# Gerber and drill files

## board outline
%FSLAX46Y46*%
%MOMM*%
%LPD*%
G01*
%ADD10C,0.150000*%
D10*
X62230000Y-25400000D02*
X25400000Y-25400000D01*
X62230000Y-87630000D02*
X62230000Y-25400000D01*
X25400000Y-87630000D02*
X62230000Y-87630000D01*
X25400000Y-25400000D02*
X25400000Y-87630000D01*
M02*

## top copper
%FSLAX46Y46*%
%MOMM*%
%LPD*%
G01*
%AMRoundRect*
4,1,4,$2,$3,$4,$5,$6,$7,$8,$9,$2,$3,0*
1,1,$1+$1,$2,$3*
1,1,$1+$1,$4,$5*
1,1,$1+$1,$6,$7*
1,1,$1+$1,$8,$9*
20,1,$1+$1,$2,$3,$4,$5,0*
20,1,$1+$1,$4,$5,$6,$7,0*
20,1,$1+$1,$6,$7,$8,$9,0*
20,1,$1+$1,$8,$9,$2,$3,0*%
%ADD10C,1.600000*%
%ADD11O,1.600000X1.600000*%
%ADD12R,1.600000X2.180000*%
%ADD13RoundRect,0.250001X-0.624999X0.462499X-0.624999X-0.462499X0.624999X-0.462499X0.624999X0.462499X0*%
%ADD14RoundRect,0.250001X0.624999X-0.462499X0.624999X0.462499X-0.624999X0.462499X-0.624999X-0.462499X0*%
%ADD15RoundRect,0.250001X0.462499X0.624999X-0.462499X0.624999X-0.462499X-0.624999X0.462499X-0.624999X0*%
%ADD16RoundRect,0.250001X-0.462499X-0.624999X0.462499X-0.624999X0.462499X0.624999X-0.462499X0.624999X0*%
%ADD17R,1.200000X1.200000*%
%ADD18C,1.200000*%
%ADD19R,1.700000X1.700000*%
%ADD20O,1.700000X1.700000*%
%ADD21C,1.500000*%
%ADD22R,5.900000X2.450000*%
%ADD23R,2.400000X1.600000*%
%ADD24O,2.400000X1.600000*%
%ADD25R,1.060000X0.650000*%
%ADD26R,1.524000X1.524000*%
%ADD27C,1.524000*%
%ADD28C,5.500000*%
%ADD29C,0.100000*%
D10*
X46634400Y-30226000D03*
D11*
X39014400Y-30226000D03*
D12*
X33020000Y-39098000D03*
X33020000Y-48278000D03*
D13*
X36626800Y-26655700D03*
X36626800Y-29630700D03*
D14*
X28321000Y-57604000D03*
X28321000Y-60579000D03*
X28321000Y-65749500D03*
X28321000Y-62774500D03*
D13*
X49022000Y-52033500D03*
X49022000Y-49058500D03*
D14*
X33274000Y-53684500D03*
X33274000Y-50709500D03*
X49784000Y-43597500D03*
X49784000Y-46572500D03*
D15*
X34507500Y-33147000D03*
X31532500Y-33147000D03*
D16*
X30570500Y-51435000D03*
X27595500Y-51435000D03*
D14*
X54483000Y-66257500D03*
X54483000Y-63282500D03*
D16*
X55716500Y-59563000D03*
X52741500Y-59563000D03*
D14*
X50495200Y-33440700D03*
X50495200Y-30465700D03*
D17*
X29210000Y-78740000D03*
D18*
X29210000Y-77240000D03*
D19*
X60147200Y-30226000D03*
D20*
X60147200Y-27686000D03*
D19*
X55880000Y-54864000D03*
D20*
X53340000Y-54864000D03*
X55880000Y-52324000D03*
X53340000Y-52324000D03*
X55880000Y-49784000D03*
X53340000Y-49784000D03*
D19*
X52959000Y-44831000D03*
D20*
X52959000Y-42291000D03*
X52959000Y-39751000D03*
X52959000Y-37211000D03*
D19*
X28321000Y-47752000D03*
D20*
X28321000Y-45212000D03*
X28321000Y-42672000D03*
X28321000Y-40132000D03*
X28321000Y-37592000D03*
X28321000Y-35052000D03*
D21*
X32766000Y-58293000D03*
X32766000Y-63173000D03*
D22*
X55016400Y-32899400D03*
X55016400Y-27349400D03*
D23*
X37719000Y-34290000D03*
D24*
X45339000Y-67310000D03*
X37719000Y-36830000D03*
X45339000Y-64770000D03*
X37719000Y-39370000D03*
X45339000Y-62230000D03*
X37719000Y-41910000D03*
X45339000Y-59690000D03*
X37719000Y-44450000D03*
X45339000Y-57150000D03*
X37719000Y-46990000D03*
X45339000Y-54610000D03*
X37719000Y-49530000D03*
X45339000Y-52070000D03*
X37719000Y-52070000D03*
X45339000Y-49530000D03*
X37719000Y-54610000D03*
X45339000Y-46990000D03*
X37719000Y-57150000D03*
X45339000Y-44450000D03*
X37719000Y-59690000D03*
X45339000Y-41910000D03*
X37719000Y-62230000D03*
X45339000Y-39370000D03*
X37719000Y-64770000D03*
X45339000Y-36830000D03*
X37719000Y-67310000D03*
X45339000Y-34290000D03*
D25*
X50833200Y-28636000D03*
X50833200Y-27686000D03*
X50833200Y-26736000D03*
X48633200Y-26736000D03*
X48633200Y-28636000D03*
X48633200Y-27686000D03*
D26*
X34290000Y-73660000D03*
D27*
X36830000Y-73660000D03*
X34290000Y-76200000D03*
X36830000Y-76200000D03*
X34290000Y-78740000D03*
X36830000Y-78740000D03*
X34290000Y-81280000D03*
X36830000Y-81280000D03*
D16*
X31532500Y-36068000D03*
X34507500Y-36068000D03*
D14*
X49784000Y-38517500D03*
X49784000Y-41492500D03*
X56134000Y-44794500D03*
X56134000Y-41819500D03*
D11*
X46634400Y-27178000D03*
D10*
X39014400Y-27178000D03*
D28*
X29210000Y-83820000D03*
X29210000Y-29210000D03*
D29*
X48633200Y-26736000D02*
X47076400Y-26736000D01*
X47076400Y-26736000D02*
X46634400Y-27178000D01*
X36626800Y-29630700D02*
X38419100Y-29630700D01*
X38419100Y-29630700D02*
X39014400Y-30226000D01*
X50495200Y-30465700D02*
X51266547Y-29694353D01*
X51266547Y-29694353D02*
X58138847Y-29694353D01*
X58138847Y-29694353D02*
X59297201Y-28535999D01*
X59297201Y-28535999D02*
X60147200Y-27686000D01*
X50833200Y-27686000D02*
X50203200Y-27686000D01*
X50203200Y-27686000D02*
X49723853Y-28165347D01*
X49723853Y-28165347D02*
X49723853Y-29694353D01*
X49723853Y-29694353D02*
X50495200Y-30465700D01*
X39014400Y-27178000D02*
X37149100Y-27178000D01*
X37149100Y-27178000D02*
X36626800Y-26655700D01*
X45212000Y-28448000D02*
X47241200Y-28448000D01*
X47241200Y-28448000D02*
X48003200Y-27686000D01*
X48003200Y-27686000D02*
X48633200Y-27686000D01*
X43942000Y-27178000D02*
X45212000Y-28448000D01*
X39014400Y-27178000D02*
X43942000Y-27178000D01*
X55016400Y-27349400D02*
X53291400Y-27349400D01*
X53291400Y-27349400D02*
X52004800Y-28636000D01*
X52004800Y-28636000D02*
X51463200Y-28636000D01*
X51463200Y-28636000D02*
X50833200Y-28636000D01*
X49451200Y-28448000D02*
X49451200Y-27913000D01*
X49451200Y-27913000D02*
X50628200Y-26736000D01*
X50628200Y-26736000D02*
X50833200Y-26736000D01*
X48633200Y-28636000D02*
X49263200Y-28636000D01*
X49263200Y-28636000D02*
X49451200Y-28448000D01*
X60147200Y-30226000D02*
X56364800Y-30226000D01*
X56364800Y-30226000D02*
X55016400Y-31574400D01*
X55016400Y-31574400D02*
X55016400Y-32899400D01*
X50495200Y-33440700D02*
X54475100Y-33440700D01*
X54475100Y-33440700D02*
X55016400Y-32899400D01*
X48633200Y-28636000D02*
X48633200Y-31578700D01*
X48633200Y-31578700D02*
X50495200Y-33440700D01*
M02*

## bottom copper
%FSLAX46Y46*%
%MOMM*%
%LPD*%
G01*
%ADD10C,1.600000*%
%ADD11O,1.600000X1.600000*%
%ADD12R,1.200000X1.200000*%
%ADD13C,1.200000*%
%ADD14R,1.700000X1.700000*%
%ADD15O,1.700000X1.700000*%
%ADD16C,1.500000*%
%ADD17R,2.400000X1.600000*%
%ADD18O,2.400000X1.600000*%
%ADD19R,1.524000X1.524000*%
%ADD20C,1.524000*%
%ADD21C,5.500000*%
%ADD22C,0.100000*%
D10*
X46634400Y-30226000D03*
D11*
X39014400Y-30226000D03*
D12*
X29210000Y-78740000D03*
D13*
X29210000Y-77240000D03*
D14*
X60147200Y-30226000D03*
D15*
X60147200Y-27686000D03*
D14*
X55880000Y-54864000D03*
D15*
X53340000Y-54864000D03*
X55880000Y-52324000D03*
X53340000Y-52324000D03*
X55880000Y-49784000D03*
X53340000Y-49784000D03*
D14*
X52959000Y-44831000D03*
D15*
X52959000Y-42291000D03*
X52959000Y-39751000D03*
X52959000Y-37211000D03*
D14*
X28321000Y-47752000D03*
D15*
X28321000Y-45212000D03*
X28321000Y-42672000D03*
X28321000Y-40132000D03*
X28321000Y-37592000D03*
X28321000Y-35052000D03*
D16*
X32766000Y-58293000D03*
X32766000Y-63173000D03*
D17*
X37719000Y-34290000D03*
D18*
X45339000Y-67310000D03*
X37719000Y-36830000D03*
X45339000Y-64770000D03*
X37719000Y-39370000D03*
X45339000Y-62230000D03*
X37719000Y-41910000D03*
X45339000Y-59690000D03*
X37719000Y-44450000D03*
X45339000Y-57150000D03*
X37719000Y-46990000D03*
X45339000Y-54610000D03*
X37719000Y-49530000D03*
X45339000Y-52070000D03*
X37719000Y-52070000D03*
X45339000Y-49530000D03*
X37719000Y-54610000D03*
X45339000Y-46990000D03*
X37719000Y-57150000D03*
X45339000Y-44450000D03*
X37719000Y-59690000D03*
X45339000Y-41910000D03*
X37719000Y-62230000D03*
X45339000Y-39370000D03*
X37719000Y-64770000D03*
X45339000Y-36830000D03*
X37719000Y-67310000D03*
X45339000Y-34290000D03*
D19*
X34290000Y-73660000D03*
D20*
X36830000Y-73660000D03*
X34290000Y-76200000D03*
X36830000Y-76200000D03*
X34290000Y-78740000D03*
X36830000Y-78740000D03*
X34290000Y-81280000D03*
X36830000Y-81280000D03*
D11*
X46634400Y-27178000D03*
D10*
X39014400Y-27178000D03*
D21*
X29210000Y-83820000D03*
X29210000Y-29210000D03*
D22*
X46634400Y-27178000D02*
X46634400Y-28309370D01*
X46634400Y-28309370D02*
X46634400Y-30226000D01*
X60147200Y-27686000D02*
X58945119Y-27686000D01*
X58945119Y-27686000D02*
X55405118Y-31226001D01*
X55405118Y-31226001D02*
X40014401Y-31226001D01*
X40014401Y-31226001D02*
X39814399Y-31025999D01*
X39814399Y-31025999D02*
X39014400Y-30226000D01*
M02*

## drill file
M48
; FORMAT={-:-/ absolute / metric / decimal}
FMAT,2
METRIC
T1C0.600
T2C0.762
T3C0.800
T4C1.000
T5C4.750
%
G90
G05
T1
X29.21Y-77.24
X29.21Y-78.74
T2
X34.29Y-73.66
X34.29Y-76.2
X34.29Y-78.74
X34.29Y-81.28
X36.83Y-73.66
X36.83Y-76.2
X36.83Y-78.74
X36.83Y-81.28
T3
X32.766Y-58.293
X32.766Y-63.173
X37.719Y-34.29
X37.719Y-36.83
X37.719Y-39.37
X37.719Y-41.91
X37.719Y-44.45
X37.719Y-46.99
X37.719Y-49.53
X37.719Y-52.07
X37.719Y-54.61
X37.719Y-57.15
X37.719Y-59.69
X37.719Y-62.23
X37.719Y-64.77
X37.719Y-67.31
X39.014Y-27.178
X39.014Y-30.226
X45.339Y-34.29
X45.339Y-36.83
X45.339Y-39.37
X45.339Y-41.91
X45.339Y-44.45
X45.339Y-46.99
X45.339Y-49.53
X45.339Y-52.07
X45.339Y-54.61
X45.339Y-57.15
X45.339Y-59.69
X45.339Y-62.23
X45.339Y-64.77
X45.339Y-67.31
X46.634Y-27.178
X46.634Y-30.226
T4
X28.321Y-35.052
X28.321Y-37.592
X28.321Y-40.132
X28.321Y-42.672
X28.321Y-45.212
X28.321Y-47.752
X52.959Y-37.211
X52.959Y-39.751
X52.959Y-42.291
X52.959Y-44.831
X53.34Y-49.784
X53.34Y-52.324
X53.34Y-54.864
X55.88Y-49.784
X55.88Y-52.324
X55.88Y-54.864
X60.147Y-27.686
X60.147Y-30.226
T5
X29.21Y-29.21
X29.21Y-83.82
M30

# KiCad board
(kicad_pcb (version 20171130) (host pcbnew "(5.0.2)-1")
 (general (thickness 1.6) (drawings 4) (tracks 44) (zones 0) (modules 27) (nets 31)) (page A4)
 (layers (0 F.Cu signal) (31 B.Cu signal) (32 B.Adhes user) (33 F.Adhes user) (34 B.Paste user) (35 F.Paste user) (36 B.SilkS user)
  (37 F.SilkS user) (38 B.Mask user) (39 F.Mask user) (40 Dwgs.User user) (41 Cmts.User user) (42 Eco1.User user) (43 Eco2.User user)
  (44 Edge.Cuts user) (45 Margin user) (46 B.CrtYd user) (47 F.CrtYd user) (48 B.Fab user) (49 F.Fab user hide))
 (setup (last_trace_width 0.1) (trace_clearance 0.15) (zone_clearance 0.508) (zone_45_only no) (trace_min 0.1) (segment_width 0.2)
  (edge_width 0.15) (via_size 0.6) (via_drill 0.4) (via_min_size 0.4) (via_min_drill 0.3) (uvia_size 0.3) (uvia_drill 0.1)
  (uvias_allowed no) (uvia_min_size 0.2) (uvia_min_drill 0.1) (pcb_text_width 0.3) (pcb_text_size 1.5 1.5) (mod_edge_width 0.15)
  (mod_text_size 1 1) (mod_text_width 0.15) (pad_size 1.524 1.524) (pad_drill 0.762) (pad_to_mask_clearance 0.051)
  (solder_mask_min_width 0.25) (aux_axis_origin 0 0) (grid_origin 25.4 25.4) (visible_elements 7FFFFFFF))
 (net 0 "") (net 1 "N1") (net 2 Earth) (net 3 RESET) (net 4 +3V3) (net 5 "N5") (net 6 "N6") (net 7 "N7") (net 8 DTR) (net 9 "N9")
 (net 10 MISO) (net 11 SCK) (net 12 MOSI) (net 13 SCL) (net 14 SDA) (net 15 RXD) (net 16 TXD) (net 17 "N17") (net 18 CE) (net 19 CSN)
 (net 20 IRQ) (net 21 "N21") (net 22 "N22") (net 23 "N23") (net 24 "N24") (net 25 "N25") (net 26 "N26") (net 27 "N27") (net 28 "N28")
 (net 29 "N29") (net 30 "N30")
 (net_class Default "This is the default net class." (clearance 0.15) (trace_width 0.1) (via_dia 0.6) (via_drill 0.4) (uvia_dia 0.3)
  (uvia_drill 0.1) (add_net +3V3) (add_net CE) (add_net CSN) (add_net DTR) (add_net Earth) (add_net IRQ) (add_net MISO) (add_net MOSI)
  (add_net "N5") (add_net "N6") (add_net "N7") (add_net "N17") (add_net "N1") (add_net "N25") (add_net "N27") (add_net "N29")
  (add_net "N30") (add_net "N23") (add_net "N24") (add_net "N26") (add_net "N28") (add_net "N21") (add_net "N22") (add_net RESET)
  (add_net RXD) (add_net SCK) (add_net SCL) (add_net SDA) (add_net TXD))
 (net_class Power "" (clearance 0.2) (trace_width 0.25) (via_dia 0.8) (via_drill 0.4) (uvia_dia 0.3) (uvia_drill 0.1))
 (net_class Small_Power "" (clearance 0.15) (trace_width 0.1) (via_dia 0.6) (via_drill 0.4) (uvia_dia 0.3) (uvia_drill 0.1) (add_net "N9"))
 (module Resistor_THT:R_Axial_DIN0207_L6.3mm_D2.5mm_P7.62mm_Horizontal (layer F.Cu) (at 46.6344 30.226 180)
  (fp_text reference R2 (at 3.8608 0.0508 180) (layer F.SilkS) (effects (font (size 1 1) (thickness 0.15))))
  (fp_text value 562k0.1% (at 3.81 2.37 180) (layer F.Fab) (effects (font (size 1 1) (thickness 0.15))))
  (pad 1 thru_hole circle (at 0 0 180) (size 1.6 1.6) (drill 0.8) (layers *.Cu *.Mask) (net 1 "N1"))
  (pad 2 thru_hole oval (at 7.62 0 180) (size 1.6 1.6) (drill 0.8) (layers *.Cu *.Mask) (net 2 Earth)))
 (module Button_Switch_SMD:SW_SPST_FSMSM (layer F.Cu) (at 33.02 43.688 270)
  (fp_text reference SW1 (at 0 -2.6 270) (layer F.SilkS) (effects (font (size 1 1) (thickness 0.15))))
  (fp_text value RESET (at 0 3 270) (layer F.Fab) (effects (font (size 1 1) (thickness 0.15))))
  (pad 1 smd rect (at -4.59 0 270) (size 2.18 1.6) (layers F.Cu F.Paste F.Mask) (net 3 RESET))
  (pad 2 smd rect (at 4.59 0 270) (size 2.18 1.6) (layers F.Cu F.Paste F.Mask) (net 2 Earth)))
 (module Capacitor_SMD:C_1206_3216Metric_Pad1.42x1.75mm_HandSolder (layer F.Cu) (at 36.6268 28.1432 270)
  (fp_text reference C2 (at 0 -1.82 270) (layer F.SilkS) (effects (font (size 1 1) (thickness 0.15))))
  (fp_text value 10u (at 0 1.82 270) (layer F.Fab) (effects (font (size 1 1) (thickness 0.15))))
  (pad 1 smd roundrect (at -1.4875 0 270) (size 1.425 1.75) (layers F.Cu F.Paste F.Mask) (roundrect_rratio 0.175439) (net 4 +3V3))
  (pad 2 smd roundrect (at 1.4875 0 270) (size 1.425 1.75) (layers F.Cu F.Paste F.Mask) (roundrect_rratio 0.175439) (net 2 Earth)))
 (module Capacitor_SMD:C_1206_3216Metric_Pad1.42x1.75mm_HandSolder (layer F.Cu) (at 28.321 59.0915 90)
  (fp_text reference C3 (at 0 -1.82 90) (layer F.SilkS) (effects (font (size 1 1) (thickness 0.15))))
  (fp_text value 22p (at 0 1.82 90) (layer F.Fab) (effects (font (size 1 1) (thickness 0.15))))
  (pad 2 smd roundrect (at 1.4875 0 90) (size 1.425 1.75) (layers F.Cu F.Paste F.Mask) (roundrect_rratio 0.175439) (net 2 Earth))
  (pad 1 smd roundrect (at -1.4875 0 90) (size 1.425 1.75) (layers F.Cu F.Paste F.Mask) (roundrect_rratio 0.175439) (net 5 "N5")))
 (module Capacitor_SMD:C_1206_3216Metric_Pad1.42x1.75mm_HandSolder (layer F.Cu) (at 28.321 64.262 90)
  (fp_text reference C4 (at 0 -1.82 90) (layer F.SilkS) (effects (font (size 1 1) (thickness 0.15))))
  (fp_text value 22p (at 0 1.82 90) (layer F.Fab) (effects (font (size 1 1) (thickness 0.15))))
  (pad 1 smd roundrect (at -1.4875 0 90) (size 1.425 1.75) (layers F.Cu F.Paste F.Mask) (roundrect_rratio 0.175439) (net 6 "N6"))
  (pad 2 smd roundrect (at 1.4875 0 90) (size 1.425 1.75) (layers F.Cu F.Paste F.Mask) (roundrect_rratio 0.175439) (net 2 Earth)))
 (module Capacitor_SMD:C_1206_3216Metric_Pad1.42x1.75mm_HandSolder (layer F.Cu) (at 49.022 50.546 270)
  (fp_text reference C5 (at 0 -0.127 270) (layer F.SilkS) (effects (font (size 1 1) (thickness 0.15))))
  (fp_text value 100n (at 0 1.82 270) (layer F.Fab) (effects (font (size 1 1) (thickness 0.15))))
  (pad 2 smd roundrect (at 1.4875 0 270) (size 1.425 1.75) (layers F.Cu F.Paste F.Mask) (roundrect_rratio 0.175439) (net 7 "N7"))
  (pad 1 smd roundrect (at -1.4875 0 270) (size 1.425 1.75) (layers F.Cu F.Paste F.Mask) (roundrect_rratio 0.175439) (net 2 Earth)))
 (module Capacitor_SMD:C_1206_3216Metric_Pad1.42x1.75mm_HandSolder (layer F.Cu) (at 33.274 52.197 90)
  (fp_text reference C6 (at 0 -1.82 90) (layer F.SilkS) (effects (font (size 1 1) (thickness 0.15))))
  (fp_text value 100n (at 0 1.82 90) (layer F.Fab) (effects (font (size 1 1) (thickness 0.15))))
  (pad 1 smd roundrect (at -1.4875 0 90) (size 1.425 1.75) (layers F.Cu F.Paste F.Mask) (roundrect_rratio 0.175439) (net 4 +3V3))
  (pad 2 smd roundrect (at 1.4875 0 90) (size 1.425 1.75) (layers F.Cu F.Paste F.Mask) (roundrect_rratio 0.175439) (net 2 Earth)))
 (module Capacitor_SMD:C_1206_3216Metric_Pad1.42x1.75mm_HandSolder (layer F.Cu) (at 49.784 45.085 90)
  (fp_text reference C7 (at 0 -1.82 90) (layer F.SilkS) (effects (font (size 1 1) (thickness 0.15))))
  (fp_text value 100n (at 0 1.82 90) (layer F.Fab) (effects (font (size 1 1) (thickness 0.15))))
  (pad 2 smd roundrect (at 1.4875 0 90) (size 1.425 1.75) (layers F.Cu F.Paste F.Mask) (roundrect_rratio 0.175439) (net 4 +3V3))
  (pad 1 smd roundrect (at -1.4875 0 90) (size 1.425 1.75) (layers F.Cu F.Paste F.Mask) (roundrect_rratio 0.175439) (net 2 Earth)))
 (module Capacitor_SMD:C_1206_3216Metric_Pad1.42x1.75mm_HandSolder (layer F.Cu) (at 33.02 33.147 180)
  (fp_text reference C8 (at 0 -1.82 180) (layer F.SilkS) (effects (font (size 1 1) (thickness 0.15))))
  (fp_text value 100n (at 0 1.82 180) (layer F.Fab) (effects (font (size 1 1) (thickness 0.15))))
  (pad 1 smd roundrect (at -1.4875 0 180) (size 1.425 1.75) (layers F.Cu F.Paste F.Mask) (roundrect_rratio 0.175439) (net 3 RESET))
  (pad 2 smd roundrect (at 1.4875 0 180) (size 1.425 1.75) (layers F.Cu F.Paste F.Mask) (roundrect_rratio 0.175439) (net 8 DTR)))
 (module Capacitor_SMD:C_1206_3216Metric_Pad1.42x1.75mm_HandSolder (layer F.Cu) (at 29.083 51.435)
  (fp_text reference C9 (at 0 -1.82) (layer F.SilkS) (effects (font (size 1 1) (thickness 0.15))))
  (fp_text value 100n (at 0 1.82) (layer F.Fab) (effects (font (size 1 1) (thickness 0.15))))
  (pad 2 smd roundrect (at 1.4875 0) (size 1.425 1.75) (layers F.Cu F.Paste F.Mask) (roundrect_rratio 0.175439) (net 2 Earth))
  (pad 1 smd roundrect (at -1.4875 0) (size 1.425 1.75) (layers F.Cu F.Paste F.Mask) (roundrect_rratio 0.175439) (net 4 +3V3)))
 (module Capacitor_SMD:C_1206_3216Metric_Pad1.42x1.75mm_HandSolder (layer F.Cu) (at 54.483 64.77 90)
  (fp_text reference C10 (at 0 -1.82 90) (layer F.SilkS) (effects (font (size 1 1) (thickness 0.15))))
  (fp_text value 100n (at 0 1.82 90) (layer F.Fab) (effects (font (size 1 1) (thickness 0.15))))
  (pad 1 smd roundrect (at -1.4875 0 90) (size 1.425 1.75) (layers F.Cu F.Paste F.Mask) (roundrect_rratio 0.175439) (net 4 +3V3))
  (pad 2 smd roundrect (at 1.4875 0 90) (size 1.425 1.75) (layers F.Cu F.Paste F.Mask) (roundrect_rratio 0.175439) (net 2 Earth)))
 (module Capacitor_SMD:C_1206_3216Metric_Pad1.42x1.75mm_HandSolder (layer F.Cu) (at 54.229 59.563)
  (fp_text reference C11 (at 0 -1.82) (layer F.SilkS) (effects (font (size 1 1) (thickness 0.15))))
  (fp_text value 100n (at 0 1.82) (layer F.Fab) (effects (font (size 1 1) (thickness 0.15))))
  (pad 2 smd roundrect (at 1.4875 0) (size 1.425 1.75) (layers F.Cu F.Paste F.Mask) (roundrect_rratio 0.175439) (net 2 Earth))
  (pad 1 smd roundrect (at -1.4875 0) (size 1.425 1.75) (layers F.Cu F.Paste F.Mask) (roundrect_rratio 0.175439) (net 4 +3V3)))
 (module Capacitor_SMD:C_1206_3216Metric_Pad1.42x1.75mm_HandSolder (layer F.Cu) (at 50.4952 31.9532 90)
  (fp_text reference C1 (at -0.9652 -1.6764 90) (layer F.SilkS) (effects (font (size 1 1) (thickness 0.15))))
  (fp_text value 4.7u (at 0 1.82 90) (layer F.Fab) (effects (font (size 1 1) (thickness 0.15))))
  (pad 1 smd roundrect (at -1.4875 0 90) (size 1.425 1.75) (layers F.Cu F.Paste F.Mask) (roundrect_rratio 0.175439) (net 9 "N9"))
  (pad 2 smd roundrect (at 1.4875 0 90) (size 1.425 1.75) (layers F.Cu F.Paste F.Mask) (roundrect_rratio 0.175439) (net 2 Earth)))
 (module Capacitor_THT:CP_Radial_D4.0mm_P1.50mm (layer F.Cu) (at 29.21 78.74 90)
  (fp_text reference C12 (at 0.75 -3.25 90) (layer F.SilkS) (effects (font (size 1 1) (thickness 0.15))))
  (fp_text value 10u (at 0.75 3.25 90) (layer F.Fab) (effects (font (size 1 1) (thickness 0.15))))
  (pad 1 thru_hole rect (at 0 0 90) (size 1.2 1.2) (drill 0.6) (layers *.Cu *.Mask) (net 4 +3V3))
  (pad 2 thru_hole circle (at 1.5 0 90) (size 1.2 1.2) (drill 0.6) (layers *.Cu *.Mask) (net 2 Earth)))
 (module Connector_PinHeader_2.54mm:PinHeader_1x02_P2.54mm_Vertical (layer F.Cu) (at 60.1472 30.226 180)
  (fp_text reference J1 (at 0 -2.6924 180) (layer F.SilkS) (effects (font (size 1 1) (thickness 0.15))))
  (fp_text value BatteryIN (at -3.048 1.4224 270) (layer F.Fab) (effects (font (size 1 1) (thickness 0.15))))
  (pad 1 thru_hole rect (at 0 0 180) (size 1.7 1.7) (drill 1) (layers *.Cu *.Mask) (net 9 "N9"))
  (pad 2 thru_hole oval (at 0 2.54 180) (size 1.7 1.7) (drill 1) (layers *.Cu *.Mask) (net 2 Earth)))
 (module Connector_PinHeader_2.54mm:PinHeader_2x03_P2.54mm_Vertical (layer F.Cu) (at 55.88 54.864 180)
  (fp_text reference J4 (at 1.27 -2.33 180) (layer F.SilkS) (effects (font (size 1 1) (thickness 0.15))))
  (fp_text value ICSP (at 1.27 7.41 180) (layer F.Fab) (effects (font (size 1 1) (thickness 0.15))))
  (pad 1 thru_hole rect (at 0 0 180) (size 1.7 1.7) (drill 1) (layers *.Cu *.Mask) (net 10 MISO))
  (pad 2 thru_hole oval (at 2.54 0 180) (size 1.7 1.7) (drill 1) (layers *.Cu *.Mask) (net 4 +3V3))
  (pad 3 thru_hole oval (at 0 2.54 180) (size 1.7 1.7) (drill 1) (layers *.Cu *.Mask) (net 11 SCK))
  (pad 4 thru_hole oval (at 2.54 2.54 180) (size 1.7 1.7) (drill 1) (layers *.Cu *.Mask) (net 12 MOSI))
  (pad 5 thru_hole oval (at 0 5.08 180) (size 1.7 1.7) (drill 1) (layers *.Cu *.Mask) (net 3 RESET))
  (pad 6 thru_hole oval (at 2.54 5.08 180) (size 1.7 1.7) (drill 1) (layers *.Cu *.Mask) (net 2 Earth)))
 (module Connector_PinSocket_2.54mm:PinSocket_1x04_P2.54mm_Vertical (layer F.Cu) (at 52.959 44.831 180)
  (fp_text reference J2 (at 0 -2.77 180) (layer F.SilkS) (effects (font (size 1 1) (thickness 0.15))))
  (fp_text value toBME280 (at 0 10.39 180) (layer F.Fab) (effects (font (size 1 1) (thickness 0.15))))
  (pad 1 thru_hole rect (at 0 0 180) (size 1.7 1.7) (drill 1) (layers *.Cu *.Mask) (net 4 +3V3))
  (pad 2 thru_hole oval (at 0 2.54 180) (size 1.7 1.7) (drill 1) (layers *.Cu *.Mask) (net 2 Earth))
  (pad 3 thru_hole oval (at 0 5.08 180) (size 1.7 1.7) (drill 1) (layers *.Cu *.Mask) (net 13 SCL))
  (pad 4 thru_hole oval (at 0 7.62 180) (size 1.7 1.7) (drill 1) (layers *.Cu *.Mask) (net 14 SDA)))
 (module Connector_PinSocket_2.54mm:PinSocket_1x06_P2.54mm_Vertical (layer F.Cu) (at 28.321 47.752 180)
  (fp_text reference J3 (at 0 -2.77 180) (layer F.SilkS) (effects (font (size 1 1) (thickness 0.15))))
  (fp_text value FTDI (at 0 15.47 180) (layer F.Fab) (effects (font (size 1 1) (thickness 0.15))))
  (pad 1 thru_hole rect (at 0 0 180) (size 1.7 1.7) (drill 1) (layers *.Cu *.Mask) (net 2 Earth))
  (pad 2 thru_hole oval (at 0 2.54 180) (size 1.7 1.7) (drill 1) (layers *.Cu *.Mask) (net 2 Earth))
  (pad 3 thru_hole oval (at 0 5.08 180) (size 1.7 1.7) (drill 1) (layers *.Cu *.Mask) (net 4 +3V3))
  (pad 4 thru_hole oval (at 0 7.62 180) (size 1.7 1.7) (drill 1) (layers *.Cu *.Mask) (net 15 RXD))
  (pad 5 thru_hole oval (at 0 10.16 180) (size 1.7 1.7) (drill 1) (layers *.Cu *.Mask) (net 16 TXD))
  (pad 6 thru_hole oval (at 0 12.7 180) (size 1.7 1.7) (drill 1) (layers *.Cu *.Mask) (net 8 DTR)))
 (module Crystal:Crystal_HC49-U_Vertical (layer F.Cu) (at 32.766 58.293 270)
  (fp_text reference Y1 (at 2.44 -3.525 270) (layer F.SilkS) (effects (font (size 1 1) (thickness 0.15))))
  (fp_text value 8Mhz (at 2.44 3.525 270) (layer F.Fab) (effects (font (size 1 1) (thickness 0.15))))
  (pad 1 thru_hole circle (at 0 0 270) (size 1.5 1.5) (drill 0.8) (layers *.Cu *.Mask) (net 5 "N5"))
  (pad 2 thru_hole circle (at 4.88 0 270) (size 1.5 1.5) (drill 0.8) (layers *.Cu *.Mask) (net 6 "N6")))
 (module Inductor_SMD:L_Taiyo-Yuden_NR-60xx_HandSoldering (layer F.Cu) (at 55.0164 30.1244 90)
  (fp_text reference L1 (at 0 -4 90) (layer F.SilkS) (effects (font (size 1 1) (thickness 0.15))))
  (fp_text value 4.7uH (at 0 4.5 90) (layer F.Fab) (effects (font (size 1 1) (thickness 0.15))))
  (pad 1 smd rect (at -2.775 0 90) (size 2.45 5.9) (layers F.Cu F.Paste F.Mask) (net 9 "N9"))
  (pad 2 smd rect (at 2.775 0 90) (size 2.45 5.9) (layers F.Cu F.Paste F.Mask) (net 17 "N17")))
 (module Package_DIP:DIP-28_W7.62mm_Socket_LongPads (layer F.Cu) (at 37.719 34.29)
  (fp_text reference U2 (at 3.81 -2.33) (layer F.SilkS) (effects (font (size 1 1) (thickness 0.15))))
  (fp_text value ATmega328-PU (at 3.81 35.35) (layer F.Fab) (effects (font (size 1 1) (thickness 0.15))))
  (pad 1 thru_hole rect (at 0 0) (size 2.4 1.6) (drill 0.8) (layers *.Cu *.Mask) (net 3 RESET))
  (pad 15 thru_hole oval (at 7.62 33.02) (size 2.4 1.6) (drill 0.8) (layers *.Cu *.Mask) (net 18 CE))
  (pad 2 thru_hole oval (at 0 2.54) (size 2.4 1.6) (drill 0.8) (layers *.Cu *.Mask) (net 15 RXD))
  (pad 16 thru_hole oval (at 7.62 30.48) (size 2.4 1.6) (drill 0.8) (layers *.Cu *.Mask) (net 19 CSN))
  (pad 3 thru_hole oval (at 0 5.08) (size 2.4 1.6) (drill 0.8) (layers *.Cu *.Mask) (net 16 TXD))
  (pad 17 thru_hole oval (at 7.62 27.94) (size 2.4 1.6) (drill 0.8) (layers *.Cu *.Mask) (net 12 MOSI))
  (pad 4 thru_hole oval (at 0 7.62) (size 2.4 1.6) (drill 0.8) (layers *.Cu *.Mask) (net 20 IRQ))
  (pad 18 thru_hole oval (at 7.62 25.4) (size 2.4 1.6) (drill 0.8) (layers *.Cu *.Mask) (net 10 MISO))
  (pad 5 thru_hole oval (at 0 10.16) (size 2.4 1.6) (drill 0.8) (layers *.Cu *.Mask) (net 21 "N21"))
  (pad 19 thru_hole oval (at 7.62 22.86) (size 2.4 1.6) (drill 0.8) (layers *.Cu *.Mask) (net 11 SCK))
  (pad 6 thru_hole oval (at 0 12.7) (size 2.4 1.6) (drill 0.8) (layers *.Cu *.Mask) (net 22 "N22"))
  (pad 20 thru_hole oval (at 7.62 20.32) (size 2.4 1.6) (drill 0.8) (layers *.Cu *.Mask) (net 4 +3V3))
  (pad 7 thru_hole oval (at 0 15.24) (size 2.4 1.6) (drill 0.8) (layers *.Cu *.Mask) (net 4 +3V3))
  (pad 21 thru_hole oval (at 7.62 17.78) (size 2.4 1.6) (drill 0.8) (layers *.Cu *.Mask) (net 7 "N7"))
  (pad 8 thru_hole oval (at 0 17.78) (size 2.4 1.6) (drill 0.8) (layers *.Cu *.Mask) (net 2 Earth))
  (pad 22 thru_hole oval (at 7.62 15.24) (size 2.4 1.6) (drill 0.8) (layers *.Cu *.Mask) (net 2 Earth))
  (pad 9 thru_hole oval (at 0 20.32) (size 2.4 1.6) (drill 0.8) (layers *.Cu *.Mask) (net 5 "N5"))
  (pad 23 thru_hole oval (at 7.62 12.7) (size 2.4 1.6) (drill 0.8) (layers *.Cu *.Mask) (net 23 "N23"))
  (pad 10 thru_hole oval (at 0 22.86) (size 2.4 1.6) (drill 0.8) (layers *.Cu *.Mask) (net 6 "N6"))
  (pad 24 thru_hole oval (at 7.62 10.16) (size 2.4 1.6) (drill 0.8) (layers *.Cu *.Mask) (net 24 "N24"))
  (pad 11 thru_hole oval (at 0 25.4) (size 2.4 1.6) (drill 0.8) (layers *.Cu *.Mask) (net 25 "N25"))
  (pad 25 thru_hole oval (at 7.62 7.62) (size 2.4 1.6) (drill 0.8) (layers *.Cu *.Mask) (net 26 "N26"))
  (pad 12 thru_hole oval (at 0 27.94) (size 2.4 1.6) (drill 0.8) (layers *.Cu *.Mask) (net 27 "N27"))
  (pad 26 thru_hole oval (at 7.62 5.08) (size 2.4 1.6) (drill 0.8) (layers *.Cu *.Mask) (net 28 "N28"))
  (pad 13 thru_hole oval (at 0 30.48) (size 2.4 1.6) (drill 0.8) (layers *.Cu *.Mask) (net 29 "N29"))
  (pad 27 thru_hole oval (at 7.62 2.54) (size 2.4 1.6) (drill 0.8) (layers *.Cu *.Mask) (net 14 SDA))
  (pad 14 thru_hole oval (at 0 33.02) (size 2.4 1.6) (drill 0.8) (layers *.Cu *.Mask) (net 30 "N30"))
  (pad 28 thru_hole oval (at 7.62 0) (size 2.4 1.6) (drill 0.8) (layers *.Cu *.Mask) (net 13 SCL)))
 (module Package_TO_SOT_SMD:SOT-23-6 (layer F.Cu) (at 49.7332 27.686 180)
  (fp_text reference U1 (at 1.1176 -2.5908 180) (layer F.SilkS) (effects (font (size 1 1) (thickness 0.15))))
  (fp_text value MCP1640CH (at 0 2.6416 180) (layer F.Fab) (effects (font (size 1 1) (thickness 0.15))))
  (pad 1 smd rect (at -1.1 -0.95 180) (size 1.06 0.65) (layers F.Cu F.Paste F.Mask) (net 17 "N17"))
  (pad 2 smd rect (at -1.1 0 180) (size 1.06 0.65) (layers F.Cu F.Paste F.Mask) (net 2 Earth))
  (pad 3 smd rect (at -1.1 0.95 180) (size 1.06 0.65) (layers F.Cu F.Paste F.Mask) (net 9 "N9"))
  (pad 4 smd rect (at 1.1 0.95 180) (size 1.06 0.65) (layers F.Cu F.Paste F.Mask) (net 1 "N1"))
  (pad 6 smd rect (at 1.1 -0.95 180) (size 1.06 0.65) (layers F.Cu F.Paste F.Mask) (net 9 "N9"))
  (pad 5 smd rect (at 1.1 0 180) (size 1.06 0.65) (layers F.Cu F.Paste F.Mask) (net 4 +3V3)))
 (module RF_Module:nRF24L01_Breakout (layer F.Cu) (at 34.29 73.66)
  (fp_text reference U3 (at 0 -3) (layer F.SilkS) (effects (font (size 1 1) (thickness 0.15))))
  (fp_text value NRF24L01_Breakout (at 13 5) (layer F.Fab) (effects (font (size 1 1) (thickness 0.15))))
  (pad 1 thru_hole rect (at 0 0) (size 1.524 1.524) (drill 0.762) (layers *.Cu *.Mask) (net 2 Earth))
  (pad 2 thru_hole circle (at 2.54 0) (size 1.524 1.524) (drill 0.762) (layers *.Cu *.Mask) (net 4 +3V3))
  (pad 3 thru_hole circle (at 0 2.54) (size 1.524 1.524) (drill 0.762) (layers *.Cu *.Mask) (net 18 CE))
  (pad 4 thru_hole circle (at 2.54 2.54) (size 1.524 1.524) (drill 0.762) (layers *.Cu *.Mask) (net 19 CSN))
  (pad 5 thru_hole circle (at 0 5.08) (size 1.524 1.524) (drill 0.762) (layers *.Cu *.Mask) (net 11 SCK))
  (pad 6 thru_hole circle (at 2.54 5.08) (size 1.524 1.524) (drill 0.762) (layers *.Cu *.Mask) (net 12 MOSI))
  (pad 7 thru_hole circle (at 0 7.62) (size 1.524 1.524) (drill 0.762) (layers *.Cu *.Mask) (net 10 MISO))
  (pad 8 thru_hole circle (at 2.54 7.62) (size 1.524 1.524) (drill 0.762) (layers *.Cu *.Mask) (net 20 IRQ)))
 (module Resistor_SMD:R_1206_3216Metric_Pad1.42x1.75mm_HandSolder (layer F.Cu) (at 33.02 36.068)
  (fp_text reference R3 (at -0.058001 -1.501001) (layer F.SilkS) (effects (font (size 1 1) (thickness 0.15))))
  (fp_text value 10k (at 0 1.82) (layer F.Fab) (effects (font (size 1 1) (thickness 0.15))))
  (pad 1 smd roundrect (at -1.4875 0) (size 1.425 1.75) (layers F.Cu F.Paste F.Mask) (roundrect_rratio 0.175439) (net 4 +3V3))
  (pad 2 smd roundrect (at 1.4875 0) (size 1.425 1.75) (layers F.Cu F.Paste F.Mask) (roundrect_rratio 0.175439) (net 3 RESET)))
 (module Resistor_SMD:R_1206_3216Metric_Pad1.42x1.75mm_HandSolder (layer F.Cu) (at 49.784 40.005 90)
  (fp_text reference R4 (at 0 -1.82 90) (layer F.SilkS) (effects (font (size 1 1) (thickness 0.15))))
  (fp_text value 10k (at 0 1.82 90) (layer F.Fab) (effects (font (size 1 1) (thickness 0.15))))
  (pad 2 smd roundrect (at 1.4875 0 90) (size 1.425 1.75) (layers F.Cu F.Paste F.Mask) (roundrect_rratio 0.175439) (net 13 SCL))
  (pad 1 smd roundrect (at -1.4875 0 90) (size 1.425 1.75) (layers F.Cu F.Paste F.Mask) (roundrect_rratio 0.175439) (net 4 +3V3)))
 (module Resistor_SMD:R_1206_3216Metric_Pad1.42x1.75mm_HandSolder (layer F.Cu) (at 56.134 43.307 90)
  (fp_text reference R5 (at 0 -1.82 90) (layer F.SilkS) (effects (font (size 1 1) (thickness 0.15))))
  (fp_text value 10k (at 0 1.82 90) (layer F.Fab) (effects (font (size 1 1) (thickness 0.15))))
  (pad 1 smd roundrect (at -1.4875 0 90) (size 1.425 1.75) (layers F.Cu F.Paste F.Mask) (roundrect_rratio 0.175439) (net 4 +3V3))
  (pad 2 smd roundrect (at 1.4875 0 90) (size 1.425 1.75) (layers F.Cu F.Paste F.Mask) (roundrect_rratio 0.175439) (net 14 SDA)))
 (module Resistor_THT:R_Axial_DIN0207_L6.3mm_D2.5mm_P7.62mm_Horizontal (layer F.Cu) (at 39.0144 27.178)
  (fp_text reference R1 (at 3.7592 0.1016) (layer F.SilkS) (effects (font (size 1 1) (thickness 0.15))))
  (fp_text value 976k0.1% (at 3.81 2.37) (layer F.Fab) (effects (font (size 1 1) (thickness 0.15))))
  (pad 2 thru_hole oval (at 7.62 0) (size 1.6 1.6) (drill 0.8) (layers *.Cu *.Mask) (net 1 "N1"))
  (pad 1 thru_hole circle (at 0 0) (size 1.6 1.6) (drill 0.8) (layers *.Cu *.Mask) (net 4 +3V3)))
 (gr_line (start 62.23 25.4) (end 25.4 25.4) (layer Edge.Cuts) (width 0.15))
 (gr_line (start 62.23 87.63) (end 62.23 25.4) (layer Edge.Cuts) (width 0.15))
 (gr_line (start 25.4 87.63) (end 62.23 87.63) (layer Edge.Cuts) (width 0.15))
 (gr_line (start 25.4 25.4) (end 25.4 87.63) (layer Edge.Cuts) (width 0.15))
 (via (at 29.21 83.82) (size 5.5) (drill 4.75) (layers F.Cu B.Cu) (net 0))
 (via (at 29.21 29.21) (size 5.5) (drill 4.75) (layers F.Cu B.Cu) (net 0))
 (segment (start 46.6344 27.178) (end 46.6344 28.30937) (width 0.1) (layer B.Cu) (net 1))
 (segment (start 46.6344 28.30937) (end 46.6344 30.226) (width 0.1) (layer B.Cu) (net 1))
 (segment (start 48.6332 26.736) (end 47.0764 26.736) (width 0.1) (layer F.Cu) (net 1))
 (segment (start 47.0764 26.736) (end 46.6344 27.178) (width 0.1) (layer F.Cu) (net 1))
 (segment (start 60.1472 27.686) (end 58.945119 27.686) (width 0.1) (layer B.Cu) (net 2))
 (segment (start 58.945119 27.686) (end 55.405118 31.226001) (width 0.1) (layer B.Cu) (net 2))
 (segment (start 55.405118 31.226001) (end 40.014401 31.226001) (width 0.1) (layer B.Cu) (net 2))
 (segment (start 40.014401 31.226001) (end 39.814399 31.025999) (width 0.1) (layer B.Cu) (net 2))
 (segment (start 39.814399 31.025999) (end 39.0144 30.226) (width 0.1) (layer B.Cu) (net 2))
 (segment (start 36.6268 29.6307) (end 38.4191 29.6307) (width 0.1) (layer F.Cu) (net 2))
 (segment (start 38.4191 29.6307) (end 39.0144 30.226) (width 0.1) (layer F.Cu) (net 2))
 (segment (start 50.4952 30.4657) (end 51.266547 29.694353) (width 0.1) (layer F.Cu) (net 2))
 (segment (start 51.266547 29.694353) (end 58.138847 29.694353) (width 0.1) (layer F.Cu) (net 2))
 (segment (start 58.138847 29.694353) (end 59.297201 28.535999) (width 0.1) (layer F.Cu) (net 2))
 (segment (start 59.297201 28.535999) (end 60.1472 27.686) (width 0.1) (layer F.Cu) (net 2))
 (segment (start 50.8332 27.686) (end 50.2032 27.686) (width 0.1) (layer F.Cu) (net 2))
 (segment (start 50.2032 27.686) (end 49.723853 28.165347) (width 0.1) (layer F.Cu) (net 2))
 (segment (start 49.723853 28.165347) (end 49.723853 29.694353) (width 0.1) (layer F.Cu) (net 2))
 (segment (start 49.723853 29.694353) (end 50.4952 30.4657) (width 0.1) (layer F.Cu) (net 2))
 (segment (start 39.0144 27.178) (end 37.1491 27.178) (width 0.1) (layer F.Cu) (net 4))
 (segment (start 37.1491 27.178) (end 36.6268 26.6557) (width 0.1) (layer F.Cu) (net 4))
 (segment (start 45.212 28.448) (end 47.2412 28.448) (width 0.1) (layer F.Cu) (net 4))
 (segment (start 47.2412 28.448) (end 48.0032 27.686) (width 0.1) (layer F.Cu) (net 4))
 (segment (start 48.0032 27.686) (end 48.6332 27.686) (width 0.1) (layer F.Cu) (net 4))
 (segment (start 43.942 27.178) (end 45.212 28.448) (width 0.1) (layer F.Cu) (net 4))
 (segment (start 39.0144 27.178) (end 43.942 27.178) (width 0.1) (layer F.Cu) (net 4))
 (segment (start 55.0164 27.3494) (end 53.2914 27.3494) (width 0.1) (layer F.Cu) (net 17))
 (segment (start 53.2914 27.3494) (end 52.0048 28.636) (width 0.1) (layer F.Cu) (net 17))
 (segment (start 52.0048 28.636) (end 51.4632 28.636) (width 0.1) (layer F.Cu) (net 17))
 (segment (start 51.4632 28.636) (end 50.8332 28.636) (width 0.1) (layer F.Cu) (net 17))
 (segment (start 49.4512 28.448) (end 49.4512 27.913) (width 0.1) (layer F.Cu) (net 9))
 (segment (start 49.4512 27.913) (end 50.6282 26.736) (width 0.1) (layer F.Cu) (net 9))
 (segment (start 50.6282 26.736) (end 50.8332 26.736) (width 0.1) (layer F.Cu) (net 9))
 (segment (start 48.6332 28.636) (end 49.2632 28.636) (width 0.1) (layer F.Cu) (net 9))
 (segment (start 49.2632 28.636) (end 49.4512 28.448) (width 0.1) (layer F.Cu) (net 9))
 (segment (start 60.1472 30.226) (end 56.3648 30.226) (width 0.1) (layer F.Cu) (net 9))
 (segment (start 56.3648 30.226) (end 55.0164 31.5744) (width 0.1) (layer F.Cu) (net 9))
 (segment (start 55.0164 31.5744) (end 55.0164 32.8994) (width 0.1) (layer F.Cu) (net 9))
 (segment (start 50.4952 33.4407) (end 54.4751 33.4407) (width 0.1) (layer F.Cu) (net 9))
 (segment (start 54.4751 33.4407) (end 55.0164 32.8994) (width 0.1) (layer F.Cu) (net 9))
 (segment (start 48.6332 28.636) (end 48.6332 31.5787) (width 0.1) (layer F.Cu) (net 9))
 (segment (start 48.6332 31.5787) (end 50.4952 33.4407) (width 0.1) (layer F.Cu) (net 9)))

